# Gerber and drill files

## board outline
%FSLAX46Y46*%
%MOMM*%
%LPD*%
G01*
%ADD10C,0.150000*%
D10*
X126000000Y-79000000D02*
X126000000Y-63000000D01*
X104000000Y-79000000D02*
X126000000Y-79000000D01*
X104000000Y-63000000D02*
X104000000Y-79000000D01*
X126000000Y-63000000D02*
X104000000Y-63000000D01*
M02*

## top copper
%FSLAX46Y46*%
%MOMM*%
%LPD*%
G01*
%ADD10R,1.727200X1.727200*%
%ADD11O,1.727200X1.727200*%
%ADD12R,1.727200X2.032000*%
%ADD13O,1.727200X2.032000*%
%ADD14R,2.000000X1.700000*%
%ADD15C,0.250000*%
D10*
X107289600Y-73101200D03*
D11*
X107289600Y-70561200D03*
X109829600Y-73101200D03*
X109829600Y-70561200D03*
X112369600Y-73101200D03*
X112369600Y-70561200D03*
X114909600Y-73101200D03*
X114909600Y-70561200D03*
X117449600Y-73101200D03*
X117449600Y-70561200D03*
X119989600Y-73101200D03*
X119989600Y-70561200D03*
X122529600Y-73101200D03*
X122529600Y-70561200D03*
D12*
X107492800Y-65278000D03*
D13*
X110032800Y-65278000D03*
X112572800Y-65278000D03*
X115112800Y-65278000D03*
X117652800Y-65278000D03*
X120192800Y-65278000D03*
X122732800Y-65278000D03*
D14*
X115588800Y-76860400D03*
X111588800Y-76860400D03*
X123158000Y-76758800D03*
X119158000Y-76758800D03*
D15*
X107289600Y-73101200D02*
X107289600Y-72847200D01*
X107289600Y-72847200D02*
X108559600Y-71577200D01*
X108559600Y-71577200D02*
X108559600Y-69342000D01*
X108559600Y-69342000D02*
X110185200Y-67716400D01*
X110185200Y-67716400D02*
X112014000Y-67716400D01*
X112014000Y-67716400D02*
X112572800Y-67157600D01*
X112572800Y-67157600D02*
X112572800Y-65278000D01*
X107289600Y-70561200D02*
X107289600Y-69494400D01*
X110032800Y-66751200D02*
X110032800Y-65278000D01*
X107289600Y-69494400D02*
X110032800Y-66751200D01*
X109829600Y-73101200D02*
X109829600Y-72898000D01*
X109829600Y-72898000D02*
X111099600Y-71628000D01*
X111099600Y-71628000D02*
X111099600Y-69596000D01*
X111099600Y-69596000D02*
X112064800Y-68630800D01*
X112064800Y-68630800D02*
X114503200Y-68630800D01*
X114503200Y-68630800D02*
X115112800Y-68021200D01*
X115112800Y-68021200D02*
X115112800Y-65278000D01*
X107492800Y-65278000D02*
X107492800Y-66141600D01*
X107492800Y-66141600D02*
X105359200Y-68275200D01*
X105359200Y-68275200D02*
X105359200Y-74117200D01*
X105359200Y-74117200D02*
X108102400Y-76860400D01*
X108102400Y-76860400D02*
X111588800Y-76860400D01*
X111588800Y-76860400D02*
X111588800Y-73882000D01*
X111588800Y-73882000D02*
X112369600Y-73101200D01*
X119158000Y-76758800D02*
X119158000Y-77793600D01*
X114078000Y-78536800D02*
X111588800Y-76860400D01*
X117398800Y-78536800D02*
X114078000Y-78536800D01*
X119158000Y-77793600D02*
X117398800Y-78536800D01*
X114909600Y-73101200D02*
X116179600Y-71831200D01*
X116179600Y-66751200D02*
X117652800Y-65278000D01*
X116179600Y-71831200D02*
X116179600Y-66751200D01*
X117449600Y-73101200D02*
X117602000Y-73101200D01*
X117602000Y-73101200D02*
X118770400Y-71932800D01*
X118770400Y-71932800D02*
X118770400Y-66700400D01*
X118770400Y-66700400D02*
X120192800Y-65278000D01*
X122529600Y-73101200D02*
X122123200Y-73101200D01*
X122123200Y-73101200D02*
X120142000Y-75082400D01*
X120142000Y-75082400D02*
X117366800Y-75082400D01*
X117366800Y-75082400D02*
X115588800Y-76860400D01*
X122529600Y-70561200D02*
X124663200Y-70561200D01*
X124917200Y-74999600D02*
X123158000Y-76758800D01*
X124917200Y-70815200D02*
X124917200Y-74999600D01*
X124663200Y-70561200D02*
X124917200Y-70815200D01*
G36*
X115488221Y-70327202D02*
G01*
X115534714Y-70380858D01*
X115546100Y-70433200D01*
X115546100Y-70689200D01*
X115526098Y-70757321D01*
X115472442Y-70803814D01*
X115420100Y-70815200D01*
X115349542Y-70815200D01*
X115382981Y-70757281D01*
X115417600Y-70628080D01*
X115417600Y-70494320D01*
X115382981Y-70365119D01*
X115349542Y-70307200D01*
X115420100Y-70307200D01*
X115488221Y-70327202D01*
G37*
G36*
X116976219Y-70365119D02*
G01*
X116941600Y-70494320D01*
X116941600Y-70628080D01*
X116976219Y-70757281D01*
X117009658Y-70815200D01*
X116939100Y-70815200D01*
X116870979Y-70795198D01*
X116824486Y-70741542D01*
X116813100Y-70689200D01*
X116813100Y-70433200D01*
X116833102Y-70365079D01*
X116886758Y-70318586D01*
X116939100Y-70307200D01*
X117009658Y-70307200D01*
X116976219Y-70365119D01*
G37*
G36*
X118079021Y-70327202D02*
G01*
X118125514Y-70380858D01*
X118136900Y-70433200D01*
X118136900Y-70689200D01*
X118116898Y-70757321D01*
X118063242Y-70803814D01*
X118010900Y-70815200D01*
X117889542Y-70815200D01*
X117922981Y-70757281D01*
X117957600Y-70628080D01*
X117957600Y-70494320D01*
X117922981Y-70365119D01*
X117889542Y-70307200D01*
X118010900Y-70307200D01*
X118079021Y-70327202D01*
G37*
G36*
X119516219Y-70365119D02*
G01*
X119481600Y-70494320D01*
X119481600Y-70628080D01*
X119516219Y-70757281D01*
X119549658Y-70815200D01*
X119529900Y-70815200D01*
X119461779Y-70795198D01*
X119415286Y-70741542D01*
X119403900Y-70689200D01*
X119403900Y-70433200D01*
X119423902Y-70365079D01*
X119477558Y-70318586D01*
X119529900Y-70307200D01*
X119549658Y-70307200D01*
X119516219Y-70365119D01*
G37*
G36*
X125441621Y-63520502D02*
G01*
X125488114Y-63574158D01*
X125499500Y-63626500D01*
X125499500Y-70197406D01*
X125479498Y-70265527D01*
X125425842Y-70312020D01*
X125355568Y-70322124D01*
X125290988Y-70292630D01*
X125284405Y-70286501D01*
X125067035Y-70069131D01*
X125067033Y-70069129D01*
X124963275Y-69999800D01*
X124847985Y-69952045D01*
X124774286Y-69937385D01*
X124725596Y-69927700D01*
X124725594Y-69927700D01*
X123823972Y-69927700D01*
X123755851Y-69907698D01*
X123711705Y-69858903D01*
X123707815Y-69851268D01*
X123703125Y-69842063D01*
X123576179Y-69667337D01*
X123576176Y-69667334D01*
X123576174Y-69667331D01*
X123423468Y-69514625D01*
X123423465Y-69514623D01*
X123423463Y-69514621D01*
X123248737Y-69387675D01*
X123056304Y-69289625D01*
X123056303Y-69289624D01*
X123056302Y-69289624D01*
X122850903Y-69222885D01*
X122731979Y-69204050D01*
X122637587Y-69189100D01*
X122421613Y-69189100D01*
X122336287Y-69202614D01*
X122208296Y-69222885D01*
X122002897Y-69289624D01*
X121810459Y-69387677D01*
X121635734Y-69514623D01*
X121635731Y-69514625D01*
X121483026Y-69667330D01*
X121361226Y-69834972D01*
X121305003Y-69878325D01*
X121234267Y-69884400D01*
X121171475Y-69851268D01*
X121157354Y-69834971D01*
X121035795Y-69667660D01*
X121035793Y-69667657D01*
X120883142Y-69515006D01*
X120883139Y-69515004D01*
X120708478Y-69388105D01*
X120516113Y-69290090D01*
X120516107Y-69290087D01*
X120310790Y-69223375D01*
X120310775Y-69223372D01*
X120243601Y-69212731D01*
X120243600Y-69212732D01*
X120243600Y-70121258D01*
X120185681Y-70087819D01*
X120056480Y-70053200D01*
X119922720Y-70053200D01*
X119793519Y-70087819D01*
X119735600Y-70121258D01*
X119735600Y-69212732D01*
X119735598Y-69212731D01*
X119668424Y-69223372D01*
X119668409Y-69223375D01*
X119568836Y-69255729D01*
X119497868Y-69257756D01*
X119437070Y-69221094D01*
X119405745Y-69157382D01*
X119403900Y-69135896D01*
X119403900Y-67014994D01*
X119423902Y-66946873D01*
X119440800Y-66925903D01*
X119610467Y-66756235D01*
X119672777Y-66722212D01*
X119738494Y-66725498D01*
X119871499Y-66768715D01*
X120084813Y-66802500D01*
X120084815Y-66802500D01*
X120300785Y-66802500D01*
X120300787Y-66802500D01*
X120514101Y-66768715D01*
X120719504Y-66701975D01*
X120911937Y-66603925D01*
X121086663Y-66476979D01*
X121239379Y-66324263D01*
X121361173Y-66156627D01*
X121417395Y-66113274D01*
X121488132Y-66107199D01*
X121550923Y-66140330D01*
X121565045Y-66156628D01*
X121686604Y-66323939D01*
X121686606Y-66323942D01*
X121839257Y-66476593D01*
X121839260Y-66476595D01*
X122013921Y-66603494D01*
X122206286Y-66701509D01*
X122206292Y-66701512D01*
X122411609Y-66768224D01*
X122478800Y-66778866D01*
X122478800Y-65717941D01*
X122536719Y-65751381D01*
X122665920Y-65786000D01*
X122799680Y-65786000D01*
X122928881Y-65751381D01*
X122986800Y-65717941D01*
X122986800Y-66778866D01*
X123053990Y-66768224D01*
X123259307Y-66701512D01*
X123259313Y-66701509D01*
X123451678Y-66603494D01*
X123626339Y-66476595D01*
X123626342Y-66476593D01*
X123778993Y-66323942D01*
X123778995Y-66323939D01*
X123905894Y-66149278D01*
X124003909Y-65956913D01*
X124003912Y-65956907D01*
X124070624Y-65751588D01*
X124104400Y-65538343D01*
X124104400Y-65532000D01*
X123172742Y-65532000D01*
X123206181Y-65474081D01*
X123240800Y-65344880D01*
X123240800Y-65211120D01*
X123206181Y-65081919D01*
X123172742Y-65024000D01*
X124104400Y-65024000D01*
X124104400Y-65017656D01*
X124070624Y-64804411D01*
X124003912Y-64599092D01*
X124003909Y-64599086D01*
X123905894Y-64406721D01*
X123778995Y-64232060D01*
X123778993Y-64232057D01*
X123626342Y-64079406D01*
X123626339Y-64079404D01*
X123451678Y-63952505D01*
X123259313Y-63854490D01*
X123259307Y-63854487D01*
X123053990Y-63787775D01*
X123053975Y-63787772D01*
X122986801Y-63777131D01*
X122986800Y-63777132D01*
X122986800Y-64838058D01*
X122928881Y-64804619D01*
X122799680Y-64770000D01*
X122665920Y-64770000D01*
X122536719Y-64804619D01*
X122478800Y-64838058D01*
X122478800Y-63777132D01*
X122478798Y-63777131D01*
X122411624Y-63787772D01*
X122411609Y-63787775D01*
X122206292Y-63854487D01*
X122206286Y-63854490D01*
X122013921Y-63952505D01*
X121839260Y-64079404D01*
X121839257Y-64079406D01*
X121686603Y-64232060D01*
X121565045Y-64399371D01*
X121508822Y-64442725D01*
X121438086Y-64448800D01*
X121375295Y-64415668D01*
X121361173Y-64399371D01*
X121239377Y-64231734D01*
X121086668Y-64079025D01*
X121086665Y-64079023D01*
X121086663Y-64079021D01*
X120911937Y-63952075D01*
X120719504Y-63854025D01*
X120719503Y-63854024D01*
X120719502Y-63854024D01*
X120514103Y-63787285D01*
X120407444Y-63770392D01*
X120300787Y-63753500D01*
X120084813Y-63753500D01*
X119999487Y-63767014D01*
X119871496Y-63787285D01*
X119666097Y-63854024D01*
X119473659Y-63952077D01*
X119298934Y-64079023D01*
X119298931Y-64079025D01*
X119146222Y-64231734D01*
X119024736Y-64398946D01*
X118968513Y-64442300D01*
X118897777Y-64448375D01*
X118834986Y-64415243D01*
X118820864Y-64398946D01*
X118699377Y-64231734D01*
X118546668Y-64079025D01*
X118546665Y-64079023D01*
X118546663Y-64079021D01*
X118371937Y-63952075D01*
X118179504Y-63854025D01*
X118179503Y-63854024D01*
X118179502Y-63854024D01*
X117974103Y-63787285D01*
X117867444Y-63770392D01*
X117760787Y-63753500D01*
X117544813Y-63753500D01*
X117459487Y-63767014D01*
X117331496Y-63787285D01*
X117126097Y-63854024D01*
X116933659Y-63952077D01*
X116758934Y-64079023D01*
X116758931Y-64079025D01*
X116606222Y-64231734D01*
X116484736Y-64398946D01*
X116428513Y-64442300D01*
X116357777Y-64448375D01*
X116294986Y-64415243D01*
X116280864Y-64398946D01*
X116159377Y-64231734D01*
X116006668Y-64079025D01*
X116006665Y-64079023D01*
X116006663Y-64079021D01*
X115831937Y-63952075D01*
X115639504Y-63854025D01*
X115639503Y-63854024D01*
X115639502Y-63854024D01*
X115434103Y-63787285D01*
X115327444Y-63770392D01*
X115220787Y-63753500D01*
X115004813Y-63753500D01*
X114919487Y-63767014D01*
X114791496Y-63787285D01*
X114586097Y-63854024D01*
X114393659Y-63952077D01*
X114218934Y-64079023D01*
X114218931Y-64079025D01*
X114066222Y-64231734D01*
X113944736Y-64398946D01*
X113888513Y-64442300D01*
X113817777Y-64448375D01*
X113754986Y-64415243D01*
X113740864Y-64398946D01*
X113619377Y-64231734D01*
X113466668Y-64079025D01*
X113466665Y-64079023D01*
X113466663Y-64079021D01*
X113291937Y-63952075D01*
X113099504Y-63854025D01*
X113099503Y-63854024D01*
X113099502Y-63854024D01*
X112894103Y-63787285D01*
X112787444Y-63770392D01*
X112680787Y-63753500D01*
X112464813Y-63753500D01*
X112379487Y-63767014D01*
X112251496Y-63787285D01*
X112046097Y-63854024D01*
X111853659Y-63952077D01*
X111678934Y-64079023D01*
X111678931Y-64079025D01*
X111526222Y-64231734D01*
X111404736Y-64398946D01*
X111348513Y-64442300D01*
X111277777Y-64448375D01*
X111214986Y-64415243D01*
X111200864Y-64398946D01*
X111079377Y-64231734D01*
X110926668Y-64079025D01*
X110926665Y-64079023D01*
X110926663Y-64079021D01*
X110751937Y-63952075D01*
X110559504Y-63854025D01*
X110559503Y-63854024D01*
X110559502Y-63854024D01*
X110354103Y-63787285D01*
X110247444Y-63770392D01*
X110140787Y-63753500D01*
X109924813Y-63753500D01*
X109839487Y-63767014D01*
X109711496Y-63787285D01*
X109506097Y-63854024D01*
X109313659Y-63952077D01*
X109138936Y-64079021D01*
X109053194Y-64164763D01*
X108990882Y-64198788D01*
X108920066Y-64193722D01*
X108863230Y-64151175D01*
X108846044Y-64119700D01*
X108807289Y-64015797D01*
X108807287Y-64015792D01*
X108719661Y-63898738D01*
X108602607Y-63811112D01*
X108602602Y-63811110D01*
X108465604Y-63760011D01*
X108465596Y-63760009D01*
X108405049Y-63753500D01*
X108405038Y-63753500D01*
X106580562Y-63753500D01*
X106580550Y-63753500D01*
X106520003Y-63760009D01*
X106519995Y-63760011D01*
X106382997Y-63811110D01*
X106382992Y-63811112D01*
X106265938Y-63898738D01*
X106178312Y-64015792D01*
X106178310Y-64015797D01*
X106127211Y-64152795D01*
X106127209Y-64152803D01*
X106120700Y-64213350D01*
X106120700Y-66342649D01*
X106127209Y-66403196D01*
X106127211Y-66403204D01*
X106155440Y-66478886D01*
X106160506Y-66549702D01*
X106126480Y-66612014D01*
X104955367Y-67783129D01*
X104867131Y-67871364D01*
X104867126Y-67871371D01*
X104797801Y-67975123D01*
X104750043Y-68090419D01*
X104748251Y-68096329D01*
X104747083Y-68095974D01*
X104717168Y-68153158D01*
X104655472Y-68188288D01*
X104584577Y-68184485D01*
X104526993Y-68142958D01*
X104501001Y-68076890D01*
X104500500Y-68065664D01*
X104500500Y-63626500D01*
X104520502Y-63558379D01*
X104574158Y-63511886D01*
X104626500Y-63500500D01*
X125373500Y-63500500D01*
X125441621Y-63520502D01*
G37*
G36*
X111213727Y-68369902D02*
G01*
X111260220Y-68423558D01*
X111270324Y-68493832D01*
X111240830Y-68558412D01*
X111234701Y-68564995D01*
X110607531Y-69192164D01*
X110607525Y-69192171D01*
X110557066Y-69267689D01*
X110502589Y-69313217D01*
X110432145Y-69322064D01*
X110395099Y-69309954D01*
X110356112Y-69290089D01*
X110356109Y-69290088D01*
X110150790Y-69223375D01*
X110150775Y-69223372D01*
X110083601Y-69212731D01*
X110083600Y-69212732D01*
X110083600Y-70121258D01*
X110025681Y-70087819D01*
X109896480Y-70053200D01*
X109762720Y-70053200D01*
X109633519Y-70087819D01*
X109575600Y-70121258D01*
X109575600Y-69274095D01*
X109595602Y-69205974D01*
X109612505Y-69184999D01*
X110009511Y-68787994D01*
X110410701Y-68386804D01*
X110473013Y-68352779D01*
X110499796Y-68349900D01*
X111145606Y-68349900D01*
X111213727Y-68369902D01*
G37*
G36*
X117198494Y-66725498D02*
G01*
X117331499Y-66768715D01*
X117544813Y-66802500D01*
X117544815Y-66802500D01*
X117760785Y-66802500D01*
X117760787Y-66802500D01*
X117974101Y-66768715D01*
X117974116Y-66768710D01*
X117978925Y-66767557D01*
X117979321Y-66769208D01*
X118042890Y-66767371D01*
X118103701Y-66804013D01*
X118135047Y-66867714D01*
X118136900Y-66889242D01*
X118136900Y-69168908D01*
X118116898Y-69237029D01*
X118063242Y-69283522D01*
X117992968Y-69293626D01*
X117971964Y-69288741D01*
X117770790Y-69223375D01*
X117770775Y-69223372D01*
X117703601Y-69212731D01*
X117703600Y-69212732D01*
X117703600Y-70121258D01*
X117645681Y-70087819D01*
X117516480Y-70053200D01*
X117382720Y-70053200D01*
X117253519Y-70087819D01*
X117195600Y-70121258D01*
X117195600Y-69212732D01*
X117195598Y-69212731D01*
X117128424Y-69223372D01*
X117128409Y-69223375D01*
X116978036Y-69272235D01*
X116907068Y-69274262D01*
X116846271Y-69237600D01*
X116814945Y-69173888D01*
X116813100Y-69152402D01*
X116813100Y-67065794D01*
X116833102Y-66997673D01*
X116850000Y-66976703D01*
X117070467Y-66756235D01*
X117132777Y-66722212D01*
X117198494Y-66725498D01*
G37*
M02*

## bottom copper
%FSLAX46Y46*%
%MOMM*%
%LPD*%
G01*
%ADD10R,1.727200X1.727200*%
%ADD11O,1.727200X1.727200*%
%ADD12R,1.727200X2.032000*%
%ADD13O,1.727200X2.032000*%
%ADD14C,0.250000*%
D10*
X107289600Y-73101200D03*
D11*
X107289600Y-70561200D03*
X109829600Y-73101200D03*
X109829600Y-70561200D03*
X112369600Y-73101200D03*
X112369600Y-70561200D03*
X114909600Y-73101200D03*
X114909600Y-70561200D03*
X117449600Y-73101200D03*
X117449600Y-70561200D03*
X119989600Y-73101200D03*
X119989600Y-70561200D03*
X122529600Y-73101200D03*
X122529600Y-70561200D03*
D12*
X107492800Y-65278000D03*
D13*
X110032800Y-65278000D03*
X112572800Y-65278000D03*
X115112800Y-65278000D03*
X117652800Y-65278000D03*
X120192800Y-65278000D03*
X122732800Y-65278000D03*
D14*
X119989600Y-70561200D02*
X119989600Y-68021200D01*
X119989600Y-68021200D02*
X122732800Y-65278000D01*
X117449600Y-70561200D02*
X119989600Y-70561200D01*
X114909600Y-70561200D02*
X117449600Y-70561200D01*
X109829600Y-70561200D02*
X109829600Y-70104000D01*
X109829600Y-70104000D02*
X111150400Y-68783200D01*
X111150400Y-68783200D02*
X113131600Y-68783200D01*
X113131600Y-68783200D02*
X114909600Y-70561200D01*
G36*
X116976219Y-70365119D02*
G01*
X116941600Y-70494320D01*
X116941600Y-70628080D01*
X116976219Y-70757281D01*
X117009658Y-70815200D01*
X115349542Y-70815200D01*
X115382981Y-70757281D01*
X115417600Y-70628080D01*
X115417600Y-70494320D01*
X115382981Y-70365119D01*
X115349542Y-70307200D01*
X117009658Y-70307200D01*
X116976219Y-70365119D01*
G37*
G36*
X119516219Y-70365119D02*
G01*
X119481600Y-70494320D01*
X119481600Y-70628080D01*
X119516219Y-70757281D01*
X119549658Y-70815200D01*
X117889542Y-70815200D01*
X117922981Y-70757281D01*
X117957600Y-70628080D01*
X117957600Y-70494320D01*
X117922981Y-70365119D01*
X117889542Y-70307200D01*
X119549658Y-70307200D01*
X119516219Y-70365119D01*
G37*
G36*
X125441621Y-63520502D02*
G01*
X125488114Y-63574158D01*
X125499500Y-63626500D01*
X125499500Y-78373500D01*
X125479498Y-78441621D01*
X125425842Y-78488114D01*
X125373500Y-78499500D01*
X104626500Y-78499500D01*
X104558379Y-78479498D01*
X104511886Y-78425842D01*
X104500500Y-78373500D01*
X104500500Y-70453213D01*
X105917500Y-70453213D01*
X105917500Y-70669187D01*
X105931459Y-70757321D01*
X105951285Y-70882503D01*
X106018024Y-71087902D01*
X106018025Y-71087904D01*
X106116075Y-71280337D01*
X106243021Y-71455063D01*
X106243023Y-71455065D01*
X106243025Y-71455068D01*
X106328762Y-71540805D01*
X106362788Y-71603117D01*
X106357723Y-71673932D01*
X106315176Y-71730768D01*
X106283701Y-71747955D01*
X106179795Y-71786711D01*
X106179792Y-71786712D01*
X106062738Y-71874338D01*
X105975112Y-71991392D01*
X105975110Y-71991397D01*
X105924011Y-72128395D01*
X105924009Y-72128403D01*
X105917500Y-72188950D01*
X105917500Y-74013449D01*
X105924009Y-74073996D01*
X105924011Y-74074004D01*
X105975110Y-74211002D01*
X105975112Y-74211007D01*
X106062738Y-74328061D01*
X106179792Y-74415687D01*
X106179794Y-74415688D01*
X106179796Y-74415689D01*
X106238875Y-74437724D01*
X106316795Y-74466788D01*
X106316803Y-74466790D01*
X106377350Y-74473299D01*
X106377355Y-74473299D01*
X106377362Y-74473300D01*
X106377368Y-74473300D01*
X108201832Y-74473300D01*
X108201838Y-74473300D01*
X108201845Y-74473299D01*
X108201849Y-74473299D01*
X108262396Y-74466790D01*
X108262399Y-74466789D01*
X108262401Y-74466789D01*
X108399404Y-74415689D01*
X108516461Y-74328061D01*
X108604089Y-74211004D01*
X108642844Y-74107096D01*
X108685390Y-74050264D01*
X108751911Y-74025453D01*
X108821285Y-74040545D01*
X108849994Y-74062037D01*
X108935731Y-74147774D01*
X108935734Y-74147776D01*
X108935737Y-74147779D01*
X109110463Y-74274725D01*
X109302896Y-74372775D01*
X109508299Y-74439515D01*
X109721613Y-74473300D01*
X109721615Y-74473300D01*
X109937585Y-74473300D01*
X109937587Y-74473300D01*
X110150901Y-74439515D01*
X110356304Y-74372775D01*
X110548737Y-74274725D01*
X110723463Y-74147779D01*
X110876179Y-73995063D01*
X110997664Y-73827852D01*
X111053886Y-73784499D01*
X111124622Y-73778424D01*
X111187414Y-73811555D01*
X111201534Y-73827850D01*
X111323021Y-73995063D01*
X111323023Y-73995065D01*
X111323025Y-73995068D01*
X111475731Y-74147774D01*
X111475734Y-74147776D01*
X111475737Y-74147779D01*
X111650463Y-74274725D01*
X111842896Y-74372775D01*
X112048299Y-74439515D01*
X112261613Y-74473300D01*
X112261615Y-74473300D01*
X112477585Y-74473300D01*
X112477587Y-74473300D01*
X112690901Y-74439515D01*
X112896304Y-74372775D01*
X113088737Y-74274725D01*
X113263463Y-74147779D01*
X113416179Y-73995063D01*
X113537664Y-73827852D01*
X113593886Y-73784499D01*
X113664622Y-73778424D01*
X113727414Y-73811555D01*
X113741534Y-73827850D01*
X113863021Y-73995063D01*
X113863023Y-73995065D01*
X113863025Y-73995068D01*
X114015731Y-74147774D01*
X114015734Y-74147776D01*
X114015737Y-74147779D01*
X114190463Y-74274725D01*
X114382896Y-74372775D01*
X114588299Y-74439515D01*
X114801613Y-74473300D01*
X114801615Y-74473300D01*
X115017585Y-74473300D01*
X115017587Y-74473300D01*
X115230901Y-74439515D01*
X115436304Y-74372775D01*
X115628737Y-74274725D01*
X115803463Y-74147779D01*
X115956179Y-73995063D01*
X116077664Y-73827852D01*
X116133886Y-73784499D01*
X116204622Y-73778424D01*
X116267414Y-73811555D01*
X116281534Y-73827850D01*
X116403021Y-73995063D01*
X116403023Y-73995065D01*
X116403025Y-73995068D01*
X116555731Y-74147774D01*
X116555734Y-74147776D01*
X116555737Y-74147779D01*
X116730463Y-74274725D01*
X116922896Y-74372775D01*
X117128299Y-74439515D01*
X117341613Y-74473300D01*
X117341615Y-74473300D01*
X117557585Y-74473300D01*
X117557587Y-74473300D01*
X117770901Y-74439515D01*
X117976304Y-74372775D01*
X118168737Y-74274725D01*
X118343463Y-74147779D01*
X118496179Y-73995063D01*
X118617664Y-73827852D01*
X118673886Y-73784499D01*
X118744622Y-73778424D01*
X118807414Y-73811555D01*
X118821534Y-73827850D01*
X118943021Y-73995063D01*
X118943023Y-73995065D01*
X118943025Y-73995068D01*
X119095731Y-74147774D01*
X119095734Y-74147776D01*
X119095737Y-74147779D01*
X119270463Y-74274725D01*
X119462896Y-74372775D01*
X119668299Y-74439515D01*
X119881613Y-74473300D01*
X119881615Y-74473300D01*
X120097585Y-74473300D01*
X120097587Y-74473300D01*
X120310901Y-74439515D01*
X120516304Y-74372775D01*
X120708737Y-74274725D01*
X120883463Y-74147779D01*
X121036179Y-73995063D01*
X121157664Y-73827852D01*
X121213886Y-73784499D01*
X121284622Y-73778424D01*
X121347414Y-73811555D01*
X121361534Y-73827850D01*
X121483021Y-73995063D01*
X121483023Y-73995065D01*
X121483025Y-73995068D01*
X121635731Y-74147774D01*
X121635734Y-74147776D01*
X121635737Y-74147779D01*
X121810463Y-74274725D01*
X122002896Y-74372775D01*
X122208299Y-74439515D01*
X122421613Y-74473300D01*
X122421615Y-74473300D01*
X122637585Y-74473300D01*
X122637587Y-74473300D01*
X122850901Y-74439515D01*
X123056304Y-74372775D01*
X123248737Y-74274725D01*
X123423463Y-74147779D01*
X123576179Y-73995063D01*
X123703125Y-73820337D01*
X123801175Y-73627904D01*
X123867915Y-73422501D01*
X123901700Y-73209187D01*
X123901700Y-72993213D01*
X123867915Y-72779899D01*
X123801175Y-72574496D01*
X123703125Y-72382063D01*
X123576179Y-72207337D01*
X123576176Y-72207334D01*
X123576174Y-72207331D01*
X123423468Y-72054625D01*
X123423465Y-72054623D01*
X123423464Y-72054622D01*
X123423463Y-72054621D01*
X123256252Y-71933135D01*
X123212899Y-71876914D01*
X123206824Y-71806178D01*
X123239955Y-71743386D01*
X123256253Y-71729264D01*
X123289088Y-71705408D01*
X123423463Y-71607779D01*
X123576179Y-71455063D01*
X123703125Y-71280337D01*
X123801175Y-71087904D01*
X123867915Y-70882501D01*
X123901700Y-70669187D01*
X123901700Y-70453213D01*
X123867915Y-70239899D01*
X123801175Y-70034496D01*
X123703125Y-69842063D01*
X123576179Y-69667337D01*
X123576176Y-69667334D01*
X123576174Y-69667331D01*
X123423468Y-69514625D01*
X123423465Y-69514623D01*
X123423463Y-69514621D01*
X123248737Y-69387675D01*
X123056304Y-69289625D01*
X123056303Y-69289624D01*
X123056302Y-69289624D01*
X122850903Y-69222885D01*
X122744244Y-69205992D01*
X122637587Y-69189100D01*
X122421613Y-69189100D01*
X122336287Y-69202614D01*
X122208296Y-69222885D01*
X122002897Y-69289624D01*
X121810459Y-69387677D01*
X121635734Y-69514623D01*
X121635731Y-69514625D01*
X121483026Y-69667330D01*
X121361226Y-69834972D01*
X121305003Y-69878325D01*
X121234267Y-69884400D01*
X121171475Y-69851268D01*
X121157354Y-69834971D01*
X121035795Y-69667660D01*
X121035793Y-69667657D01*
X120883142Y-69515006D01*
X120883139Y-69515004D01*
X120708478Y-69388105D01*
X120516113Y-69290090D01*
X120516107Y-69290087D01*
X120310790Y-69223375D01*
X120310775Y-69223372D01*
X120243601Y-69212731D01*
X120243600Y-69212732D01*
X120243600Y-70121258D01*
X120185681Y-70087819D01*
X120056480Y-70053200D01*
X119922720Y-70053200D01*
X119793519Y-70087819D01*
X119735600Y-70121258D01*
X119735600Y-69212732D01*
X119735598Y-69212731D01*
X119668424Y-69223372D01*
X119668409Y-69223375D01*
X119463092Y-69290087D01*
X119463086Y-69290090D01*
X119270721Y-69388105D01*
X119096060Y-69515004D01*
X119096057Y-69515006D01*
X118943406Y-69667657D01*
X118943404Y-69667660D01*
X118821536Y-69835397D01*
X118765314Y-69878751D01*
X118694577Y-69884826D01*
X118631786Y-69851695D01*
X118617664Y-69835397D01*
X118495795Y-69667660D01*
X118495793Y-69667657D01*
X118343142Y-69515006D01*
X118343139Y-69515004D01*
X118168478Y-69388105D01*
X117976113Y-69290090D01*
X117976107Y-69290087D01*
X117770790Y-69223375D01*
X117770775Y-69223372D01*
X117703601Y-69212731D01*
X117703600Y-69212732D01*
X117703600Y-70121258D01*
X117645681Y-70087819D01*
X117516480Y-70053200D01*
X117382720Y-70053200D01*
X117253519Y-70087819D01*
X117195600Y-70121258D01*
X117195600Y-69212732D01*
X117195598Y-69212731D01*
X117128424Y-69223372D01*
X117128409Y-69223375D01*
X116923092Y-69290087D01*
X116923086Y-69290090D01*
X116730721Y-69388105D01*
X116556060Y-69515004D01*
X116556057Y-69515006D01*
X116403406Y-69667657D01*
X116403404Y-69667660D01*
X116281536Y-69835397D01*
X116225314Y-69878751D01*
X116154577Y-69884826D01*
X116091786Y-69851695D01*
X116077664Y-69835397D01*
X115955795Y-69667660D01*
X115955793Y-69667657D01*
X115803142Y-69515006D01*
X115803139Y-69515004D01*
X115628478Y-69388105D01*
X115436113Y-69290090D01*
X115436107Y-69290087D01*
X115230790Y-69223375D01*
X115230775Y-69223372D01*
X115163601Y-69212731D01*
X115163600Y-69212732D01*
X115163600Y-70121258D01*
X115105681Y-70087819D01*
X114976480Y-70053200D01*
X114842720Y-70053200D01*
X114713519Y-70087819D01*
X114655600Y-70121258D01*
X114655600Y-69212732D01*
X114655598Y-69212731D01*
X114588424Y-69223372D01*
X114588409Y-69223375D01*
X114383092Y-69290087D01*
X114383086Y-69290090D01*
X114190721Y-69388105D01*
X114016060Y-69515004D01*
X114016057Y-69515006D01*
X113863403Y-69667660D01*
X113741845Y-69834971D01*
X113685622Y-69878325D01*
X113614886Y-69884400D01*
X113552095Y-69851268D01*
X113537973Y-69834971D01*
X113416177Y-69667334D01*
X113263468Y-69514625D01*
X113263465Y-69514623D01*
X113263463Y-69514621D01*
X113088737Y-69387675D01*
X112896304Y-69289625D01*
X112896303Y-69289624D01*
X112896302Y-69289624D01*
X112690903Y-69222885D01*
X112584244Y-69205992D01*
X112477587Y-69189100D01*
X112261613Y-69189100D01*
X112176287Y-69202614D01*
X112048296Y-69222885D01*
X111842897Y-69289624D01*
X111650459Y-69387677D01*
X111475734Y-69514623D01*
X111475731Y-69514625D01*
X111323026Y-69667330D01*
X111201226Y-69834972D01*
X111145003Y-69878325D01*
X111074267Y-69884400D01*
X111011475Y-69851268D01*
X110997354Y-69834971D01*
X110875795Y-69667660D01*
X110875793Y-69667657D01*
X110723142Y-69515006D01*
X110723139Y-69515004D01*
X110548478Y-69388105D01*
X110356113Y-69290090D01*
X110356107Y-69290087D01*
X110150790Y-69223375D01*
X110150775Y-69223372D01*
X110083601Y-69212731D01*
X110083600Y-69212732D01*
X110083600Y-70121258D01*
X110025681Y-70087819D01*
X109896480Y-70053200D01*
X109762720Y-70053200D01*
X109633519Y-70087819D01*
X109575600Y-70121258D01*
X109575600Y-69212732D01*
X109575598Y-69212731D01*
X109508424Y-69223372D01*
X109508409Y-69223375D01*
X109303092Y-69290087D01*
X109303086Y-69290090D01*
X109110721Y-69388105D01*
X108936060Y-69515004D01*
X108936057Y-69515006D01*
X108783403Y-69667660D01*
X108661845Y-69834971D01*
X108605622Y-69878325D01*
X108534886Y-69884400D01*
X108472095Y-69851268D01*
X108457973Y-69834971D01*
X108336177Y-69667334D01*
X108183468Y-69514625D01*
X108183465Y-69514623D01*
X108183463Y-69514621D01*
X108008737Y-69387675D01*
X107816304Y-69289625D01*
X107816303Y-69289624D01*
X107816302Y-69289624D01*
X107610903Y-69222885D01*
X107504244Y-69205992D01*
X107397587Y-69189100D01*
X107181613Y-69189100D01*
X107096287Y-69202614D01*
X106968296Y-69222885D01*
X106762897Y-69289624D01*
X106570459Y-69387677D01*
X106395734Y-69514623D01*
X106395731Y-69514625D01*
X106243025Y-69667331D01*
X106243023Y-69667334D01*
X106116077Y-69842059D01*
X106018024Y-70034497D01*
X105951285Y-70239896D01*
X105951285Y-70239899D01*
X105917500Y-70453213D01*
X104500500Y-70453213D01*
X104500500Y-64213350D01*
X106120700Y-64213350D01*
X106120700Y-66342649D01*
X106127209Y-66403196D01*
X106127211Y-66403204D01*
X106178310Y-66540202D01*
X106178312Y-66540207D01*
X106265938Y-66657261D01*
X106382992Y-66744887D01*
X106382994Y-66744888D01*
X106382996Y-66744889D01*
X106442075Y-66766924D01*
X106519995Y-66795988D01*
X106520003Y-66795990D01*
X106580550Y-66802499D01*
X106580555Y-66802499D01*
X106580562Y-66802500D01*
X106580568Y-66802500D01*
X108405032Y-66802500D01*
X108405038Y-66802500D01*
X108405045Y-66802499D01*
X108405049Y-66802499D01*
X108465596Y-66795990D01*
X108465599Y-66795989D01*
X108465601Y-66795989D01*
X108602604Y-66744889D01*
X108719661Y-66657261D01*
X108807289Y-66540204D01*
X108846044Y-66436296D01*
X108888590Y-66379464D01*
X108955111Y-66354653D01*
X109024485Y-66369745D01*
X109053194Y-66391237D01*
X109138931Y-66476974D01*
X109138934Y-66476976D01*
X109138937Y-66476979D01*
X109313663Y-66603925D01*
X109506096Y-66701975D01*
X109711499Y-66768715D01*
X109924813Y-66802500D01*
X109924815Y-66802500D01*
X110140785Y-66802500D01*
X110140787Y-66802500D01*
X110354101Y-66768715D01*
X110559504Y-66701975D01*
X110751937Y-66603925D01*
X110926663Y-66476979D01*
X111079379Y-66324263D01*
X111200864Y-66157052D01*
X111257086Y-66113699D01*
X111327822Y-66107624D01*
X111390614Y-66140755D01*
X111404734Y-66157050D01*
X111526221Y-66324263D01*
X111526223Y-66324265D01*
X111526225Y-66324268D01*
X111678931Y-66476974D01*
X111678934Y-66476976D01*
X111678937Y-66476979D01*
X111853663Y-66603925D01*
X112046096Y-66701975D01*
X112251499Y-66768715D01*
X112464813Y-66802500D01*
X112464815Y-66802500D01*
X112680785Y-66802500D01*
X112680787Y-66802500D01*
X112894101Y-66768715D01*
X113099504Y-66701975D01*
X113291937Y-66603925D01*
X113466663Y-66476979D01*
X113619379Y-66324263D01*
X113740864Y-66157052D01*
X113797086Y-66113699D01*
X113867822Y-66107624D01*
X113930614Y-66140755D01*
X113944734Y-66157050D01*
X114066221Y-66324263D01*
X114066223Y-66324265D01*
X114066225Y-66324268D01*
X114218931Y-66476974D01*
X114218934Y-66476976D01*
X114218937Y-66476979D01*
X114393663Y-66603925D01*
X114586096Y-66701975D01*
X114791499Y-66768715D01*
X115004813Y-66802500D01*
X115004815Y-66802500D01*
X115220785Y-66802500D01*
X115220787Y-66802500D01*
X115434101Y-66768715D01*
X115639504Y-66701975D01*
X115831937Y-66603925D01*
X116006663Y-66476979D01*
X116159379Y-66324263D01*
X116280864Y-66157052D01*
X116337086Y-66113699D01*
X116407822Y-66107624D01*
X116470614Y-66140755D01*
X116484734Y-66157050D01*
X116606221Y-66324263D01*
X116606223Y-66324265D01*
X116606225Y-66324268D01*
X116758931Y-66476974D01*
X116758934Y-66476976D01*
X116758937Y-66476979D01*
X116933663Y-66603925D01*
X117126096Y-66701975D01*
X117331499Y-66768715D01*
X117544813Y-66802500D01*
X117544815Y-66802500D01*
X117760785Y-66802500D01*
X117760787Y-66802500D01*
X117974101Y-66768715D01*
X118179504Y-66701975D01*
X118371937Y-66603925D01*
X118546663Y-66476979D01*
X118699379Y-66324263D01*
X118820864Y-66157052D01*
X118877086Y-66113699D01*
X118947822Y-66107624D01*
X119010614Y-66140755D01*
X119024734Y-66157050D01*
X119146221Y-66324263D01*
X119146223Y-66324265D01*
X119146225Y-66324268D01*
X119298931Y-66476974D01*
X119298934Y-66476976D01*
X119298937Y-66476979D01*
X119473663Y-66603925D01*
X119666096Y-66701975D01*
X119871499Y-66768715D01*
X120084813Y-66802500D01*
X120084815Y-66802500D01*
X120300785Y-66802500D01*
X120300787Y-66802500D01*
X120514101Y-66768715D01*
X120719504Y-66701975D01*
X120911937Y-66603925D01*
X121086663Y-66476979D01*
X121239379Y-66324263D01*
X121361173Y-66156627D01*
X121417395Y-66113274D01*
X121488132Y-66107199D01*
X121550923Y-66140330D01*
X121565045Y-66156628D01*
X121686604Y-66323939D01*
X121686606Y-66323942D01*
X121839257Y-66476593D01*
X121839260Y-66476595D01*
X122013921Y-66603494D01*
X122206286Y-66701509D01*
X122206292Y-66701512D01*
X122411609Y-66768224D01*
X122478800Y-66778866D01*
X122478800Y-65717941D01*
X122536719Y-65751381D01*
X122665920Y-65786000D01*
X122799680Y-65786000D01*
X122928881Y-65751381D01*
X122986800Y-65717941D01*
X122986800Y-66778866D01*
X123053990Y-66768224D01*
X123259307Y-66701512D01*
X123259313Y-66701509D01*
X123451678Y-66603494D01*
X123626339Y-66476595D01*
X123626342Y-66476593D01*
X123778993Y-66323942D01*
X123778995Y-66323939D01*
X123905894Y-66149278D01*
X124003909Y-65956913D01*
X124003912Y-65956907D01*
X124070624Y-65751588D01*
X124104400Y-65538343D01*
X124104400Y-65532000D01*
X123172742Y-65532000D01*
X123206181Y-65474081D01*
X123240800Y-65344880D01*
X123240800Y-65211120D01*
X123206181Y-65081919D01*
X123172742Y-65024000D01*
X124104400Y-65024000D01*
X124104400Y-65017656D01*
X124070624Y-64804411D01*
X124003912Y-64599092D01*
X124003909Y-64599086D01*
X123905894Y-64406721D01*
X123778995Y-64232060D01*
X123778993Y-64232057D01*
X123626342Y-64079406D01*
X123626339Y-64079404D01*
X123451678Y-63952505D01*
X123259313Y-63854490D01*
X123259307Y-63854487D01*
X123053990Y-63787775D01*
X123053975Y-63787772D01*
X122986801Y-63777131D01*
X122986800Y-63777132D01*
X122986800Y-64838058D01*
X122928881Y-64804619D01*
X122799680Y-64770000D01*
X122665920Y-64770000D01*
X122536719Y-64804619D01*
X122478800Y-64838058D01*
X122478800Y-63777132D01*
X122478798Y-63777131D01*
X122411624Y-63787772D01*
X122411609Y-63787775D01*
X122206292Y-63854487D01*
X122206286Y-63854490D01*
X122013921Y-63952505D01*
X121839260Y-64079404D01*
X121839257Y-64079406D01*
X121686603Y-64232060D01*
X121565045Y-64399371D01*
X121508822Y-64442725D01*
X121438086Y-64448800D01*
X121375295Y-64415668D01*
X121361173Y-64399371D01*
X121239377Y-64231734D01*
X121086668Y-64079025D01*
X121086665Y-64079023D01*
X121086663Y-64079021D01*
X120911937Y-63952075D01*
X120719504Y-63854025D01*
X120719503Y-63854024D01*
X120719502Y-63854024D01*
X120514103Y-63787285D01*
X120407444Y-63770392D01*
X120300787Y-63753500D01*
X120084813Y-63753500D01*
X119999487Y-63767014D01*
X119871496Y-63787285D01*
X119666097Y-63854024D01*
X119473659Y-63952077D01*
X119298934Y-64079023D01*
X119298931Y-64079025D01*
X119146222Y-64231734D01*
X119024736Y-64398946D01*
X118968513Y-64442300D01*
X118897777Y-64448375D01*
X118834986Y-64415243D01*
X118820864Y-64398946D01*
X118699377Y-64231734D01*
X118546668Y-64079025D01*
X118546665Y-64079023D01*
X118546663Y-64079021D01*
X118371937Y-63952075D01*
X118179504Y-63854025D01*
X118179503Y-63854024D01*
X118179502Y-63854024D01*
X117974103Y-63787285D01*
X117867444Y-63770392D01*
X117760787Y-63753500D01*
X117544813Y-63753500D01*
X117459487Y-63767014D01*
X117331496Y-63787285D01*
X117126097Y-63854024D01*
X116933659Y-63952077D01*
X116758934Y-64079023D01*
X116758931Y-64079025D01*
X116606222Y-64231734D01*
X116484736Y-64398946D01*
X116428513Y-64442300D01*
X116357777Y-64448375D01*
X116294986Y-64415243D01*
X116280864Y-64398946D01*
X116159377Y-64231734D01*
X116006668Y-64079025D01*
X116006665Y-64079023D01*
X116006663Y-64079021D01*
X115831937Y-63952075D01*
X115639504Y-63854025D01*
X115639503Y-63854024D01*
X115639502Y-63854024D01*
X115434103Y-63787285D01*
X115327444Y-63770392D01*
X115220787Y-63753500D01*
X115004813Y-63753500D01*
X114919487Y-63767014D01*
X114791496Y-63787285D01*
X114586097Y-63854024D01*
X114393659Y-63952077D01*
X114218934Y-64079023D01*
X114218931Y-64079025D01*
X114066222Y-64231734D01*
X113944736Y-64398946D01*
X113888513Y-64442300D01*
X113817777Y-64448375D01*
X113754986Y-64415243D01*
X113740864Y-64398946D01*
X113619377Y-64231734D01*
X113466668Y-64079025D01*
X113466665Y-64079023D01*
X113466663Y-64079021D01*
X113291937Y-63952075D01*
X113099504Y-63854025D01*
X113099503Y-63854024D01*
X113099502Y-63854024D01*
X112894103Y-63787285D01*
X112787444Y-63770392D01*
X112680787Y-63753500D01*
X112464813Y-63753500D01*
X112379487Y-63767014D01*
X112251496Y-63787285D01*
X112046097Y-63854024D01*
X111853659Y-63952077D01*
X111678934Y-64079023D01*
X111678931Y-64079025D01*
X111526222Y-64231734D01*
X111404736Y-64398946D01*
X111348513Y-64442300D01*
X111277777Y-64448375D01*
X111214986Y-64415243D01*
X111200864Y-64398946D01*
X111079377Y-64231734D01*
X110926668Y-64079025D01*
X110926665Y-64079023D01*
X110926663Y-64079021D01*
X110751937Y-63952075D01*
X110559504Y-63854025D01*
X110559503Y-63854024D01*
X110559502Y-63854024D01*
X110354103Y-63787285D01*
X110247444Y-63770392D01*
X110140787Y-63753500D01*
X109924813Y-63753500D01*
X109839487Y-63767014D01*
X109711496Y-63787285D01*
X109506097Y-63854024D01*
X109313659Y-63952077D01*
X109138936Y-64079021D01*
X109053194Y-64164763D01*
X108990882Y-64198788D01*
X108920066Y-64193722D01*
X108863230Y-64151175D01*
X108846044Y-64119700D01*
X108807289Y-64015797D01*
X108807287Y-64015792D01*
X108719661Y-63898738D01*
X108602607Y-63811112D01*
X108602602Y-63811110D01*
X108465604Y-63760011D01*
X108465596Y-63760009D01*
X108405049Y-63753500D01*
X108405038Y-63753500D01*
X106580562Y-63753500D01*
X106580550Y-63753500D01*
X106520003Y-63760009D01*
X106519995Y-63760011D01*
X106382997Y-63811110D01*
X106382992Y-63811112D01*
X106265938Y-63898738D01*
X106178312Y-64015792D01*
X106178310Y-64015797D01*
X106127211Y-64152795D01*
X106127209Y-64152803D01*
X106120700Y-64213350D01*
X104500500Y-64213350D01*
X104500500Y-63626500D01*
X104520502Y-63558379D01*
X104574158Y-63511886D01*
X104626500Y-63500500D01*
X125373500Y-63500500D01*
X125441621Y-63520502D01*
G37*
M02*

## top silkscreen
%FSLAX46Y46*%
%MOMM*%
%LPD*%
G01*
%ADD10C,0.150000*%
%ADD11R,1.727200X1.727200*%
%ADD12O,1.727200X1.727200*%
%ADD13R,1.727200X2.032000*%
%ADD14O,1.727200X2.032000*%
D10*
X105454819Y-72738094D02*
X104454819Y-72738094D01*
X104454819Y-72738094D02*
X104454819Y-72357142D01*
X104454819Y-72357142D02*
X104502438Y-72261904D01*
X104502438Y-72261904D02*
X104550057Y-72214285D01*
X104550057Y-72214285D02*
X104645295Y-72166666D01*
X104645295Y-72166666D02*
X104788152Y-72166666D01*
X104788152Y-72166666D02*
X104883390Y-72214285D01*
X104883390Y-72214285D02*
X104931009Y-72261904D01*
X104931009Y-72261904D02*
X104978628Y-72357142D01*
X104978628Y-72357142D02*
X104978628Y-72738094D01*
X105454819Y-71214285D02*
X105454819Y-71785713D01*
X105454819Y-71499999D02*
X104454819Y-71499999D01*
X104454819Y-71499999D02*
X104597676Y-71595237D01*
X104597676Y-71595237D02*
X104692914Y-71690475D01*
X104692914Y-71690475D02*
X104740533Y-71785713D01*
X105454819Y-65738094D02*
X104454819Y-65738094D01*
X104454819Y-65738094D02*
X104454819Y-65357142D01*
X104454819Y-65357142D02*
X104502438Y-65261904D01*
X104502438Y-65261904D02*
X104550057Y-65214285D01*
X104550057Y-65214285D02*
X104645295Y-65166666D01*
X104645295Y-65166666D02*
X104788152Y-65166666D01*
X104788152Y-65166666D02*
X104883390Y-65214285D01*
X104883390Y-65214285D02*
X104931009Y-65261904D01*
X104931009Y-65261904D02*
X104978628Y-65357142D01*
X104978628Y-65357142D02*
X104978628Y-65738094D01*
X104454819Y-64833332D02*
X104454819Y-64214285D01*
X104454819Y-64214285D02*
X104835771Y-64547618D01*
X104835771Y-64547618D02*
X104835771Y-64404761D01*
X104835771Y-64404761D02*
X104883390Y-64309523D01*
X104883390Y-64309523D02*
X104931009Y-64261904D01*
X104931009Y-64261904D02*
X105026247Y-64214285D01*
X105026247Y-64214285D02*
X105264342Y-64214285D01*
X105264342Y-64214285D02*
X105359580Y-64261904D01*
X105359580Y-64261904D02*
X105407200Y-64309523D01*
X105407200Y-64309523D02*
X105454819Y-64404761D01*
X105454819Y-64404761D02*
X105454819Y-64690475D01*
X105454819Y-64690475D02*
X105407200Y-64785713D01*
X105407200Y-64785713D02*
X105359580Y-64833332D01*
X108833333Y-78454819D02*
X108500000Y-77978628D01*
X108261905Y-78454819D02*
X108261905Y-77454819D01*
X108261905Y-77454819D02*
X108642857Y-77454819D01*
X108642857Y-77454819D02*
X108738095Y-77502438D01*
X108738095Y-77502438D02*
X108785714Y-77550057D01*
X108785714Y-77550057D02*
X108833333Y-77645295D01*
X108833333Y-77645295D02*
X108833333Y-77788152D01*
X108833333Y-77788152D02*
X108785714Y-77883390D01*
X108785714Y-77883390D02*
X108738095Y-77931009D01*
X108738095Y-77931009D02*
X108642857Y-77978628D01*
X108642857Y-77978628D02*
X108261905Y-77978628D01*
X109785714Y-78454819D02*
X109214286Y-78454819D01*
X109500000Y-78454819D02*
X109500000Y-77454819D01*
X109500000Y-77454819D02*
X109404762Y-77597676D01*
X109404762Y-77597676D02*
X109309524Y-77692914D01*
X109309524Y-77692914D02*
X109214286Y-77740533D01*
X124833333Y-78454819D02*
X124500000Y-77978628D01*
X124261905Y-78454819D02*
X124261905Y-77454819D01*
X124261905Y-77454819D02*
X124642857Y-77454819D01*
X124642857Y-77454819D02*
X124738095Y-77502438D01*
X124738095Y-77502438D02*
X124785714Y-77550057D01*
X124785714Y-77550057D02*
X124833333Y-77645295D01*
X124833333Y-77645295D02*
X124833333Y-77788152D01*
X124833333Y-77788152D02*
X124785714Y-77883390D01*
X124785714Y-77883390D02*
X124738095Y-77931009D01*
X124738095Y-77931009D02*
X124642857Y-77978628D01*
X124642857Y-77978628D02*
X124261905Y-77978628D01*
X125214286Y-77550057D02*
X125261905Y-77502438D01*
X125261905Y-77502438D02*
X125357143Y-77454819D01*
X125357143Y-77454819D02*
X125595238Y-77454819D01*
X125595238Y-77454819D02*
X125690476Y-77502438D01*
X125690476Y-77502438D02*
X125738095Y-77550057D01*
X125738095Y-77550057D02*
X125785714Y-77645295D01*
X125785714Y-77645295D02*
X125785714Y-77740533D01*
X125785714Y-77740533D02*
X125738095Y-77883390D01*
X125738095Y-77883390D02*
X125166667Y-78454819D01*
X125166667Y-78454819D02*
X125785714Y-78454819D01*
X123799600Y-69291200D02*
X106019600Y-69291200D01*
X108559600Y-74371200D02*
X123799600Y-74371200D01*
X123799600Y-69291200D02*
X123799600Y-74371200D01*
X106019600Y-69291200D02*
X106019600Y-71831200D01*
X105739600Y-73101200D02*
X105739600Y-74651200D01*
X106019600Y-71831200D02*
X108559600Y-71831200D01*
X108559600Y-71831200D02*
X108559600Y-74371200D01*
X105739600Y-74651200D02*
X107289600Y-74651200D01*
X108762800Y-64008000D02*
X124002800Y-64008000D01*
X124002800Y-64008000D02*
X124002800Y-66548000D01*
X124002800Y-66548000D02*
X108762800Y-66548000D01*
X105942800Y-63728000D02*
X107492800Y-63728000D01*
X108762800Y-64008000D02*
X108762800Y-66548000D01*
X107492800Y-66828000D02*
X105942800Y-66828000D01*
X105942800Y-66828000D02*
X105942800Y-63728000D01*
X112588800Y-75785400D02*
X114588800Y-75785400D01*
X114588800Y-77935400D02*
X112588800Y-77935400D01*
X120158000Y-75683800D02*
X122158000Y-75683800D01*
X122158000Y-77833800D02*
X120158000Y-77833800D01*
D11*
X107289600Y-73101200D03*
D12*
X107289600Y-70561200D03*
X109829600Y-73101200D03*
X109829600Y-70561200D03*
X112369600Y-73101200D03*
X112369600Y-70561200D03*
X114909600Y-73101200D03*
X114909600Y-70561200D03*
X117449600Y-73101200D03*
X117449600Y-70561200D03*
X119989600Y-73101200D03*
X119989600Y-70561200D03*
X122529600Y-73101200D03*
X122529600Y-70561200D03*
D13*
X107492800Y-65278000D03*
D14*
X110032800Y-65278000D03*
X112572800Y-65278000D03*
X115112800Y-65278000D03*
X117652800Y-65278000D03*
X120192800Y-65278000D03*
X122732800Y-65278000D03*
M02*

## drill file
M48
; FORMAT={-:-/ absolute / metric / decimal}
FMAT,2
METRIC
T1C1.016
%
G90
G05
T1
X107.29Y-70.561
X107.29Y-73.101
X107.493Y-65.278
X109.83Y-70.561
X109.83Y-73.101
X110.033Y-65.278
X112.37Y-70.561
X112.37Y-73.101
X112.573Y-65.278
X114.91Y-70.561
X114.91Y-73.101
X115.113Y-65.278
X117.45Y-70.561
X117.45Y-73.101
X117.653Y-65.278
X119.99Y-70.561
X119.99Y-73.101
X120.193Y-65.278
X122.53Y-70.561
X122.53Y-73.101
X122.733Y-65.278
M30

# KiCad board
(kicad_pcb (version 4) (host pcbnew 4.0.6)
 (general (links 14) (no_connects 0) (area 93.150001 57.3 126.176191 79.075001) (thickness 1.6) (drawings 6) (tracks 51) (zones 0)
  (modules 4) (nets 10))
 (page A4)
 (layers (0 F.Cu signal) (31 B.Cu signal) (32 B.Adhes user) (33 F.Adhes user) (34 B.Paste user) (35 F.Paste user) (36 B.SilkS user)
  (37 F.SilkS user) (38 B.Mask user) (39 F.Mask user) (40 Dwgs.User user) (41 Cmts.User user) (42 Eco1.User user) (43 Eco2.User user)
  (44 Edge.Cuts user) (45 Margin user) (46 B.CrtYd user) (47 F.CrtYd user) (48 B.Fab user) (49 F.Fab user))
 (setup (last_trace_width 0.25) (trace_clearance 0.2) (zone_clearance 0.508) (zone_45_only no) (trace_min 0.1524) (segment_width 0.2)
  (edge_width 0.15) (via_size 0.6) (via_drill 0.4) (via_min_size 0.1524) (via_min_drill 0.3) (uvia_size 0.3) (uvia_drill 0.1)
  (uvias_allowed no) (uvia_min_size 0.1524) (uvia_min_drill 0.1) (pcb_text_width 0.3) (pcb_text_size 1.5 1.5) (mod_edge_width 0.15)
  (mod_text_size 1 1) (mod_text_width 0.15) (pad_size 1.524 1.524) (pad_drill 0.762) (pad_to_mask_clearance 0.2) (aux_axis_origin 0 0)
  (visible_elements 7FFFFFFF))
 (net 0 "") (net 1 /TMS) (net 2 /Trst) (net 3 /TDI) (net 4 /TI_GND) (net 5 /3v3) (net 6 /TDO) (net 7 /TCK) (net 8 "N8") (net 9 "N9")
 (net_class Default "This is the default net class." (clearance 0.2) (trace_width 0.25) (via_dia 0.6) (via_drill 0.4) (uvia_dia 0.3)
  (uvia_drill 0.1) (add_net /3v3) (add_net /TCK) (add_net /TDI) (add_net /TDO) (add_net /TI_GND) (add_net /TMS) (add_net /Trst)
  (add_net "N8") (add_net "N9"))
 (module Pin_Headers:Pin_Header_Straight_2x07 (layer F.Cu) (at 107.2896 73.1012 90)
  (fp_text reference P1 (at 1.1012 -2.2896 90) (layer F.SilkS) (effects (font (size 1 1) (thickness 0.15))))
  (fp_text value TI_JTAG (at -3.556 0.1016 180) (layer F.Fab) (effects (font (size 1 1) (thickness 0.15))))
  (fp_line (start 3.81 16.51) (end 3.81 -1.27) (layer F.SilkS) (width 0.15))
  (fp_line (start -1.27 1.27) (end -1.27 16.51) (layer F.SilkS) (width 0.15))
  (fp_line (start 3.81 16.51) (end -1.27 16.51) (layer F.SilkS) (width 0.15))
  (fp_line (start 3.81 -1.27) (end 1.27 -1.27) (layer F.SilkS) (width 0.15))
  (fp_line (start 0 -1.55) (end -1.55 -1.55) (layer F.SilkS) (width 0.15))
  (fp_line (start 1.27 -1.27) (end 1.27 1.27) (layer F.SilkS) (width 0.15))
  (fp_line (start 1.27 1.27) (end -1.27 1.27) (layer F.SilkS) (width 0.15))
  (fp_line (start -1.55 -1.55) (end -1.55 0) (layer F.SilkS) (width 0.15))
  (pad 1 thru_hole rect (at 0 0 90) (size 1.7272 1.7272) (drill 1.016) (layers *.Cu *.Mask F.SilkS) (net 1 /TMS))
  (pad 2 thru_hole oval (at 2.54 0 90) (size 1.7272 1.7272) (drill 1.016) (layers *.Cu *.Mask F.SilkS) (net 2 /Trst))
  (pad 3 thru_hole oval (at 0 2.54 90) (size 1.7272 1.7272) (drill 1.016) (layers *.Cu *.Mask F.SilkS) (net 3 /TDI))
  (pad 4 thru_hole oval (at 2.54 2.54 90) (size 1.7272 1.7272) (drill 1.016) (layers *.Cu *.Mask F.SilkS) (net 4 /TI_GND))
  (pad 5 thru_hole oval (at 0 5.08 90) (size 1.7272 1.7272) (drill 1.016) (layers *.Cu *.Mask F.SilkS) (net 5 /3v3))
  (pad 6 thru_hole oval (at 2.54 5.08 90) (size 1.7272 1.7272) (drill 1.016) (layers *.Cu *.Mask F.SilkS))
  (pad 7 thru_hole oval (at 0 7.62 90) (size 1.7272 1.7272) (drill 1.016) (layers *.Cu *.Mask F.SilkS) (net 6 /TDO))
  (pad 8 thru_hole oval (at 2.54 7.62 90) (size 1.7272 1.7272) (drill 1.016) (layers *.Cu *.Mask F.SilkS) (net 4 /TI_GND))
  (pad 9 thru_hole oval (at 0 10.16 90) (size 1.7272 1.7272) (drill 1.016) (layers *.Cu *.Mask F.SilkS) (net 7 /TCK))
  (pad 10 thru_hole oval (at 2.54 10.16 90) (size 1.7272 1.7272) (drill 1.016) (layers *.Cu *.Mask F.SilkS) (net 4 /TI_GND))
  (pad 11 thru_hole oval (at 0 12.7 90) (size 1.7272 1.7272) (drill 1.016) (layers *.Cu *.Mask F.SilkS))
  (pad 12 thru_hole oval (at 2.54 12.7 90) (size 1.7272 1.7272) (drill 1.016) (layers *.Cu *.Mask F.SilkS) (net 4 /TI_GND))
  (pad 13 thru_hole oval (at 0 15.24 90) (size 1.7272 1.7272) (drill 1.016) (layers *.Cu *.Mask F.SilkS) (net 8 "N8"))
  (pad 14 thru_hole oval (at 2.54 15.24 90) (size 1.7272 1.7272) (drill 1.016) (layers *.Cu *.Mask F.SilkS) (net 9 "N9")))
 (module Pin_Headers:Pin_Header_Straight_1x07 (layer F.Cu) (at 107.4928 65.278 90)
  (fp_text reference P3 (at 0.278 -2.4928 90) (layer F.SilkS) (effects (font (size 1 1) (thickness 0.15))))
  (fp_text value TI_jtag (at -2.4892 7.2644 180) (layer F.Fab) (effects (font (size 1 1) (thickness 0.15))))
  (fp_line (start 1.27 1.27) (end 1.27 16.51) (layer F.SilkS) (width 0.15))
  (fp_line (start 1.27 16.51) (end -1.27 16.51) (layer F.SilkS) (width 0.15))
  (fp_line (start -1.27 16.51) (end -1.27 1.27) (layer F.SilkS) (width 0.15))
  (fp_line (start 1.55 -1.55) (end 1.55 0) (layer F.SilkS) (width 0.15))
  (fp_line (start 1.27 1.27) (end -1.27 1.27) (layer F.SilkS) (width 0.15))
  (fp_line (start -1.55 0) (end -1.55 -1.55) (layer F.SilkS) (width 0.15))
  (fp_line (start -1.55 -1.55) (end 1.55 -1.55) (layer F.SilkS) (width 0.15))
  (pad 1 thru_hole rect (at 0 0 90) (size 2.032 1.7272) (drill 1.016) (layers *.Cu *.Mask F.SilkS) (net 5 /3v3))
  (pad 2 thru_hole oval (at 0 2.54 90) (size 2.032 1.7272) (drill 1.016) (layers *.Cu *.Mask F.SilkS) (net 2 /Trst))
  (pad 3 thru_hole oval (at 0 5.08 90) (size 2.032 1.7272) (drill 1.016) (layers *.Cu *.Mask F.SilkS) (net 1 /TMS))
  (pad 4 thru_hole oval (at 0 7.62 90) (size 2.032 1.7272) (drill 1.016) (layers *.Cu *.Mask F.SilkS) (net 3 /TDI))
  (pad 5 thru_hole oval (at 0 10.16 90) (size 2.032 1.7272) (drill 1.016) (layers *.Cu *.Mask F.SilkS) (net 6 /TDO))
  (pad 6 thru_hole oval (at 0 12.7 90) (size 2.032 1.7272) (drill 1.016) (layers *.Cu *.Mask F.SilkS) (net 7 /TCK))
  (pad 7 thru_hole oval (at 0 15.24 90) (size 2.032 1.7272) (drill 1.016) (layers *.Cu *.Mask F.SilkS) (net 4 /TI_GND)))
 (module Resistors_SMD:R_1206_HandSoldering (layer F.Cu) (at 113.5888 76.8604 180)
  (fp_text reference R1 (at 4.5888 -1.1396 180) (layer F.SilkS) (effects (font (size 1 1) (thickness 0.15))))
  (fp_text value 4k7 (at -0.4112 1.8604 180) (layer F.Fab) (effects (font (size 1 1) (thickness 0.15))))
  (fp_line (start 1 1.075) (end -1 1.075) (layer F.SilkS) (width 0.15))
  (fp_line (start -1 -1.075) (end 1 -1.075) (layer F.SilkS) (width 0.15))
  (pad 1 smd rect (at -2 0 180) (size 2 1.7) (layers F.Cu F.Paste F.Mask) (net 8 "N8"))
  (pad 2 smd rect (at 2 0 180) (size 2 1.7) (layers F.Cu F.Paste F.Mask) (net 5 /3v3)))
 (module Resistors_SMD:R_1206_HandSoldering (layer F.Cu) (at 121.158 76.7588 180)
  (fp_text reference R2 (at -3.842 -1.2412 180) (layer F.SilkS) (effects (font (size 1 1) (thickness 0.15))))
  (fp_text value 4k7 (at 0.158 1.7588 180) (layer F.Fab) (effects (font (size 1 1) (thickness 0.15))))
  (fp_line (start 1 1.075) (end -1 1.075) (layer F.SilkS) (width 0.15))
  (fp_line (start -1 -1.075) (end 1 -1.075) (layer F.SilkS) (width 0.15))
  (pad 1 smd rect (at -2 0 180) (size 2 1.7) (layers F.Cu F.Paste F.Mask) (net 9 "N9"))
  (pad 2 smd rect (at 2 0 180) (size 2 1.7) (layers F.Cu F.Paste F.Mask) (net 5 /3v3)))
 (gr_line (start 126 79) (end 126 63) (angle 90) (layer Edge.Cuts) (width 0.15))
 (gr_line (start 104 79) (end 126 79) (angle 90) (layer Edge.Cuts) (width 0.15))
 (gr_line (start 104 63) (end 104 79) (angle 90) (layer Edge.Cuts) (width 0.15))
 (gr_line (start 126 63) (end 104 63) (angle 90) (layer Edge.Cuts) (width 0.15))
 (segment (start 107.2896 73.1012) (end 107.2896 72.8472) (width 0.25) (layer F.Cu) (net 1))
 (segment (start 107.2896 72.8472) (end 108.5596 71.5772) (width 0.25) (layer F.Cu) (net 1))
 (segment (start 108.5596 71.5772) (end 108.5596 69.342) (width 0.25) (layer F.Cu) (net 1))
 (segment (start 108.5596 69.342) (end 110.1852 67.7164) (width 0.25) (layer F.Cu) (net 1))
 (segment (start 110.1852 67.7164) (end 112.014 67.7164) (width 0.25) (layer F.Cu) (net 1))
 (segment (start 112.014 67.7164) (end 112.5728 67.1576) (width 0.25) (layer F.Cu) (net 1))
 (segment (start 112.5728 67.1576) (end 112.5728 65.278) (width 0.25) (layer F.Cu) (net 1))
 (segment (start 107.2896 70.5612) (end 107.2896 69.4944) (width 0.25) (layer F.Cu) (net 2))
 (segment (start 110.0328 66.7512) (end 110.0328 65.278) (width 0.25) (layer F.Cu) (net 2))
 (segment (start 107.2896 69.4944) (end 110.0328 66.7512) (width 0.25) (layer F.Cu) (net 2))
 (segment (start 109.8296 73.1012) (end 109.8296 72.898) (width 0.25) (layer F.Cu) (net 3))
 (segment (start 109.8296 72.898) (end 111.0996 71.628) (width 0.25) (layer F.Cu) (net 3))
 (segment (start 111.0996 71.628) (end 111.0996 69.596) (width 0.25) (layer F.Cu) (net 3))
 (segment (start 111.0996 69.596) (end 112.0648 68.6308) (width 0.25) (layer F.Cu) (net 3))
 (segment (start 112.0648 68.6308) (end 114.5032 68.6308) (width 0.25) (layer F.Cu) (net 3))
 (segment (start 114.5032 68.6308) (end 115.1128 68.0212) (width 0.25) (layer F.Cu) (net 3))
 (segment (start 115.1128 68.0212) (end 115.1128 65.278) (width 0.25) (layer F.Cu) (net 3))
 (segment (start 119.9896 70.5612) (end 119.9896 68.0212) (width 0.25) (layer B.Cu) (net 4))
 (segment (start 119.9896 68.0212) (end 122.7328 65.278) (width 0.25) (layer B.Cu) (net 4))
 (segment (start 117.4496 70.5612) (end 119.9896 70.5612) (width 0.25) (layer B.Cu) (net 4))
 (segment (start 114.9096 70.5612) (end 117.4496 70.5612) (width 0.25) (layer B.Cu) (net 4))
 (segment (start 109.8296 70.5612) (end 109.8296 70.104) (width 0.25) (layer B.Cu) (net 4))
 (segment (start 109.8296 70.104) (end 111.1504 68.7832) (width 0.25) (layer B.Cu) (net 4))
 (segment (start 111.1504 68.7832) (end 113.1316 68.7832) (width 0.25) (layer B.Cu) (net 4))
 (segment (start 113.1316 68.7832) (end 114.9096 70.5612) (width 0.25) (layer B.Cu) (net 4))
 (segment (start 107.4928 65.278) (end 107.4928 66.1416) (width 0.25) (layer F.Cu) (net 5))
 (segment (start 107.4928 66.1416) (end 105.3592 68.2752) (width 0.25) (layer F.Cu) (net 5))
 (segment (start 105.3592 68.2752) (end 105.3592 74.1172) (width 0.25) (layer F.Cu) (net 5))
 (segment (start 105.3592 74.1172) (end 108.1024 76.8604) (width 0.25) (layer F.Cu) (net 5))
 (segment (start 108.1024 76.8604) (end 111.5888 76.8604) (width 0.25) (layer F.Cu) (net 5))
 (segment (start 111.5888 76.8604) (end 111.5888 73.882) (width 0.25) (layer F.Cu) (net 5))
 (segment (start 111.5888 73.882) (end 112.3696 73.1012) (width 0.25) (layer F.Cu) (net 5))
 (segment (start 119.158 76.7588) (end 119.158 77.7936) (width 0.25) (layer F.Cu) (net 5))
 (segment (start 114.078 78.5368) (end 111.5888 76.8604) (width 0.25) (layer F.Cu) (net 5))
 (segment (start 117.3988 78.5368) (end 114.078 78.5368) (width 0.25) (layer F.Cu) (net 5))
 (segment (start 119.158 77.7936) (end 117.3988 78.5368) (width 0.25) (layer F.Cu) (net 5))
 (segment (start 114.9096 73.1012) (end 116.1796 71.8312) (width 0.25) (layer F.Cu) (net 6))
 (segment (start 116.1796 66.7512) (end 117.6528 65.278) (width 0.25) (layer F.Cu) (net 6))
 (segment (start 116.1796 71.8312) (end 116.1796 66.7512) (width 0.25) (layer F.Cu) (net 6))
 (segment (start 117.4496 73.1012) (end 117.602 73.1012) (width 0.25) (layer F.Cu) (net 7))
 (segment (start 117.602 73.1012) (end 118.7704 71.9328) (width 0.25) (layer F.Cu) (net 7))
 (segment (start 118.7704 71.9328) (end 118.7704 66.7004) (width 0.25) (layer F.Cu) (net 7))
 (segment (start 118.7704 66.7004) (end 120.1928 65.278) (width 0.25) (layer F.Cu) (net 7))
 (segment (start 122.5296 73.1012) (end 122.1232 73.1012) (width 0.25) (layer F.Cu) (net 8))
 (segment (start 122.1232 73.1012) (end 120.142 75.0824) (width 0.25) (layer F.Cu) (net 8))
 (segment (start 120.142 75.0824) (end 117.3668 75.0824) (width 0.25) (layer F.Cu) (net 8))
 (segment (start 117.3668 75.0824) (end 115.5888 76.8604) (width 0.25) (layer F.Cu) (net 8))
 (segment (start 122.5296 70.5612) (end 124.6632 70.5612) (width 0.25) (layer F.Cu) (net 9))
 (segment (start 124.9172 74.9996) (end 123.158 76.7588) (width 0.25) (layer F.Cu) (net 9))
 (segment (start 124.9172 70.8152) (end 124.9172 74.9996) (width 0.25) (layer F.Cu) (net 9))
 (segment (start 124.6632 70.5612) (end 124.9172 70.8152) (width 0.25) (layer F.Cu) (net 9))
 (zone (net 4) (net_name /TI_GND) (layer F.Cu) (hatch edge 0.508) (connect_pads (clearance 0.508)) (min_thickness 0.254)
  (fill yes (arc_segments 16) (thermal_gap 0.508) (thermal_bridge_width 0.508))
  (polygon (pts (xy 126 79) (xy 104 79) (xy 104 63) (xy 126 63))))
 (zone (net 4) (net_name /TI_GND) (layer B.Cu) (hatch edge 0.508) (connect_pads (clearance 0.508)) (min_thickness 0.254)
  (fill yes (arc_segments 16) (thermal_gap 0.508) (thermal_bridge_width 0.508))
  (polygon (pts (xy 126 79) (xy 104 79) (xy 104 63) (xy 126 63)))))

